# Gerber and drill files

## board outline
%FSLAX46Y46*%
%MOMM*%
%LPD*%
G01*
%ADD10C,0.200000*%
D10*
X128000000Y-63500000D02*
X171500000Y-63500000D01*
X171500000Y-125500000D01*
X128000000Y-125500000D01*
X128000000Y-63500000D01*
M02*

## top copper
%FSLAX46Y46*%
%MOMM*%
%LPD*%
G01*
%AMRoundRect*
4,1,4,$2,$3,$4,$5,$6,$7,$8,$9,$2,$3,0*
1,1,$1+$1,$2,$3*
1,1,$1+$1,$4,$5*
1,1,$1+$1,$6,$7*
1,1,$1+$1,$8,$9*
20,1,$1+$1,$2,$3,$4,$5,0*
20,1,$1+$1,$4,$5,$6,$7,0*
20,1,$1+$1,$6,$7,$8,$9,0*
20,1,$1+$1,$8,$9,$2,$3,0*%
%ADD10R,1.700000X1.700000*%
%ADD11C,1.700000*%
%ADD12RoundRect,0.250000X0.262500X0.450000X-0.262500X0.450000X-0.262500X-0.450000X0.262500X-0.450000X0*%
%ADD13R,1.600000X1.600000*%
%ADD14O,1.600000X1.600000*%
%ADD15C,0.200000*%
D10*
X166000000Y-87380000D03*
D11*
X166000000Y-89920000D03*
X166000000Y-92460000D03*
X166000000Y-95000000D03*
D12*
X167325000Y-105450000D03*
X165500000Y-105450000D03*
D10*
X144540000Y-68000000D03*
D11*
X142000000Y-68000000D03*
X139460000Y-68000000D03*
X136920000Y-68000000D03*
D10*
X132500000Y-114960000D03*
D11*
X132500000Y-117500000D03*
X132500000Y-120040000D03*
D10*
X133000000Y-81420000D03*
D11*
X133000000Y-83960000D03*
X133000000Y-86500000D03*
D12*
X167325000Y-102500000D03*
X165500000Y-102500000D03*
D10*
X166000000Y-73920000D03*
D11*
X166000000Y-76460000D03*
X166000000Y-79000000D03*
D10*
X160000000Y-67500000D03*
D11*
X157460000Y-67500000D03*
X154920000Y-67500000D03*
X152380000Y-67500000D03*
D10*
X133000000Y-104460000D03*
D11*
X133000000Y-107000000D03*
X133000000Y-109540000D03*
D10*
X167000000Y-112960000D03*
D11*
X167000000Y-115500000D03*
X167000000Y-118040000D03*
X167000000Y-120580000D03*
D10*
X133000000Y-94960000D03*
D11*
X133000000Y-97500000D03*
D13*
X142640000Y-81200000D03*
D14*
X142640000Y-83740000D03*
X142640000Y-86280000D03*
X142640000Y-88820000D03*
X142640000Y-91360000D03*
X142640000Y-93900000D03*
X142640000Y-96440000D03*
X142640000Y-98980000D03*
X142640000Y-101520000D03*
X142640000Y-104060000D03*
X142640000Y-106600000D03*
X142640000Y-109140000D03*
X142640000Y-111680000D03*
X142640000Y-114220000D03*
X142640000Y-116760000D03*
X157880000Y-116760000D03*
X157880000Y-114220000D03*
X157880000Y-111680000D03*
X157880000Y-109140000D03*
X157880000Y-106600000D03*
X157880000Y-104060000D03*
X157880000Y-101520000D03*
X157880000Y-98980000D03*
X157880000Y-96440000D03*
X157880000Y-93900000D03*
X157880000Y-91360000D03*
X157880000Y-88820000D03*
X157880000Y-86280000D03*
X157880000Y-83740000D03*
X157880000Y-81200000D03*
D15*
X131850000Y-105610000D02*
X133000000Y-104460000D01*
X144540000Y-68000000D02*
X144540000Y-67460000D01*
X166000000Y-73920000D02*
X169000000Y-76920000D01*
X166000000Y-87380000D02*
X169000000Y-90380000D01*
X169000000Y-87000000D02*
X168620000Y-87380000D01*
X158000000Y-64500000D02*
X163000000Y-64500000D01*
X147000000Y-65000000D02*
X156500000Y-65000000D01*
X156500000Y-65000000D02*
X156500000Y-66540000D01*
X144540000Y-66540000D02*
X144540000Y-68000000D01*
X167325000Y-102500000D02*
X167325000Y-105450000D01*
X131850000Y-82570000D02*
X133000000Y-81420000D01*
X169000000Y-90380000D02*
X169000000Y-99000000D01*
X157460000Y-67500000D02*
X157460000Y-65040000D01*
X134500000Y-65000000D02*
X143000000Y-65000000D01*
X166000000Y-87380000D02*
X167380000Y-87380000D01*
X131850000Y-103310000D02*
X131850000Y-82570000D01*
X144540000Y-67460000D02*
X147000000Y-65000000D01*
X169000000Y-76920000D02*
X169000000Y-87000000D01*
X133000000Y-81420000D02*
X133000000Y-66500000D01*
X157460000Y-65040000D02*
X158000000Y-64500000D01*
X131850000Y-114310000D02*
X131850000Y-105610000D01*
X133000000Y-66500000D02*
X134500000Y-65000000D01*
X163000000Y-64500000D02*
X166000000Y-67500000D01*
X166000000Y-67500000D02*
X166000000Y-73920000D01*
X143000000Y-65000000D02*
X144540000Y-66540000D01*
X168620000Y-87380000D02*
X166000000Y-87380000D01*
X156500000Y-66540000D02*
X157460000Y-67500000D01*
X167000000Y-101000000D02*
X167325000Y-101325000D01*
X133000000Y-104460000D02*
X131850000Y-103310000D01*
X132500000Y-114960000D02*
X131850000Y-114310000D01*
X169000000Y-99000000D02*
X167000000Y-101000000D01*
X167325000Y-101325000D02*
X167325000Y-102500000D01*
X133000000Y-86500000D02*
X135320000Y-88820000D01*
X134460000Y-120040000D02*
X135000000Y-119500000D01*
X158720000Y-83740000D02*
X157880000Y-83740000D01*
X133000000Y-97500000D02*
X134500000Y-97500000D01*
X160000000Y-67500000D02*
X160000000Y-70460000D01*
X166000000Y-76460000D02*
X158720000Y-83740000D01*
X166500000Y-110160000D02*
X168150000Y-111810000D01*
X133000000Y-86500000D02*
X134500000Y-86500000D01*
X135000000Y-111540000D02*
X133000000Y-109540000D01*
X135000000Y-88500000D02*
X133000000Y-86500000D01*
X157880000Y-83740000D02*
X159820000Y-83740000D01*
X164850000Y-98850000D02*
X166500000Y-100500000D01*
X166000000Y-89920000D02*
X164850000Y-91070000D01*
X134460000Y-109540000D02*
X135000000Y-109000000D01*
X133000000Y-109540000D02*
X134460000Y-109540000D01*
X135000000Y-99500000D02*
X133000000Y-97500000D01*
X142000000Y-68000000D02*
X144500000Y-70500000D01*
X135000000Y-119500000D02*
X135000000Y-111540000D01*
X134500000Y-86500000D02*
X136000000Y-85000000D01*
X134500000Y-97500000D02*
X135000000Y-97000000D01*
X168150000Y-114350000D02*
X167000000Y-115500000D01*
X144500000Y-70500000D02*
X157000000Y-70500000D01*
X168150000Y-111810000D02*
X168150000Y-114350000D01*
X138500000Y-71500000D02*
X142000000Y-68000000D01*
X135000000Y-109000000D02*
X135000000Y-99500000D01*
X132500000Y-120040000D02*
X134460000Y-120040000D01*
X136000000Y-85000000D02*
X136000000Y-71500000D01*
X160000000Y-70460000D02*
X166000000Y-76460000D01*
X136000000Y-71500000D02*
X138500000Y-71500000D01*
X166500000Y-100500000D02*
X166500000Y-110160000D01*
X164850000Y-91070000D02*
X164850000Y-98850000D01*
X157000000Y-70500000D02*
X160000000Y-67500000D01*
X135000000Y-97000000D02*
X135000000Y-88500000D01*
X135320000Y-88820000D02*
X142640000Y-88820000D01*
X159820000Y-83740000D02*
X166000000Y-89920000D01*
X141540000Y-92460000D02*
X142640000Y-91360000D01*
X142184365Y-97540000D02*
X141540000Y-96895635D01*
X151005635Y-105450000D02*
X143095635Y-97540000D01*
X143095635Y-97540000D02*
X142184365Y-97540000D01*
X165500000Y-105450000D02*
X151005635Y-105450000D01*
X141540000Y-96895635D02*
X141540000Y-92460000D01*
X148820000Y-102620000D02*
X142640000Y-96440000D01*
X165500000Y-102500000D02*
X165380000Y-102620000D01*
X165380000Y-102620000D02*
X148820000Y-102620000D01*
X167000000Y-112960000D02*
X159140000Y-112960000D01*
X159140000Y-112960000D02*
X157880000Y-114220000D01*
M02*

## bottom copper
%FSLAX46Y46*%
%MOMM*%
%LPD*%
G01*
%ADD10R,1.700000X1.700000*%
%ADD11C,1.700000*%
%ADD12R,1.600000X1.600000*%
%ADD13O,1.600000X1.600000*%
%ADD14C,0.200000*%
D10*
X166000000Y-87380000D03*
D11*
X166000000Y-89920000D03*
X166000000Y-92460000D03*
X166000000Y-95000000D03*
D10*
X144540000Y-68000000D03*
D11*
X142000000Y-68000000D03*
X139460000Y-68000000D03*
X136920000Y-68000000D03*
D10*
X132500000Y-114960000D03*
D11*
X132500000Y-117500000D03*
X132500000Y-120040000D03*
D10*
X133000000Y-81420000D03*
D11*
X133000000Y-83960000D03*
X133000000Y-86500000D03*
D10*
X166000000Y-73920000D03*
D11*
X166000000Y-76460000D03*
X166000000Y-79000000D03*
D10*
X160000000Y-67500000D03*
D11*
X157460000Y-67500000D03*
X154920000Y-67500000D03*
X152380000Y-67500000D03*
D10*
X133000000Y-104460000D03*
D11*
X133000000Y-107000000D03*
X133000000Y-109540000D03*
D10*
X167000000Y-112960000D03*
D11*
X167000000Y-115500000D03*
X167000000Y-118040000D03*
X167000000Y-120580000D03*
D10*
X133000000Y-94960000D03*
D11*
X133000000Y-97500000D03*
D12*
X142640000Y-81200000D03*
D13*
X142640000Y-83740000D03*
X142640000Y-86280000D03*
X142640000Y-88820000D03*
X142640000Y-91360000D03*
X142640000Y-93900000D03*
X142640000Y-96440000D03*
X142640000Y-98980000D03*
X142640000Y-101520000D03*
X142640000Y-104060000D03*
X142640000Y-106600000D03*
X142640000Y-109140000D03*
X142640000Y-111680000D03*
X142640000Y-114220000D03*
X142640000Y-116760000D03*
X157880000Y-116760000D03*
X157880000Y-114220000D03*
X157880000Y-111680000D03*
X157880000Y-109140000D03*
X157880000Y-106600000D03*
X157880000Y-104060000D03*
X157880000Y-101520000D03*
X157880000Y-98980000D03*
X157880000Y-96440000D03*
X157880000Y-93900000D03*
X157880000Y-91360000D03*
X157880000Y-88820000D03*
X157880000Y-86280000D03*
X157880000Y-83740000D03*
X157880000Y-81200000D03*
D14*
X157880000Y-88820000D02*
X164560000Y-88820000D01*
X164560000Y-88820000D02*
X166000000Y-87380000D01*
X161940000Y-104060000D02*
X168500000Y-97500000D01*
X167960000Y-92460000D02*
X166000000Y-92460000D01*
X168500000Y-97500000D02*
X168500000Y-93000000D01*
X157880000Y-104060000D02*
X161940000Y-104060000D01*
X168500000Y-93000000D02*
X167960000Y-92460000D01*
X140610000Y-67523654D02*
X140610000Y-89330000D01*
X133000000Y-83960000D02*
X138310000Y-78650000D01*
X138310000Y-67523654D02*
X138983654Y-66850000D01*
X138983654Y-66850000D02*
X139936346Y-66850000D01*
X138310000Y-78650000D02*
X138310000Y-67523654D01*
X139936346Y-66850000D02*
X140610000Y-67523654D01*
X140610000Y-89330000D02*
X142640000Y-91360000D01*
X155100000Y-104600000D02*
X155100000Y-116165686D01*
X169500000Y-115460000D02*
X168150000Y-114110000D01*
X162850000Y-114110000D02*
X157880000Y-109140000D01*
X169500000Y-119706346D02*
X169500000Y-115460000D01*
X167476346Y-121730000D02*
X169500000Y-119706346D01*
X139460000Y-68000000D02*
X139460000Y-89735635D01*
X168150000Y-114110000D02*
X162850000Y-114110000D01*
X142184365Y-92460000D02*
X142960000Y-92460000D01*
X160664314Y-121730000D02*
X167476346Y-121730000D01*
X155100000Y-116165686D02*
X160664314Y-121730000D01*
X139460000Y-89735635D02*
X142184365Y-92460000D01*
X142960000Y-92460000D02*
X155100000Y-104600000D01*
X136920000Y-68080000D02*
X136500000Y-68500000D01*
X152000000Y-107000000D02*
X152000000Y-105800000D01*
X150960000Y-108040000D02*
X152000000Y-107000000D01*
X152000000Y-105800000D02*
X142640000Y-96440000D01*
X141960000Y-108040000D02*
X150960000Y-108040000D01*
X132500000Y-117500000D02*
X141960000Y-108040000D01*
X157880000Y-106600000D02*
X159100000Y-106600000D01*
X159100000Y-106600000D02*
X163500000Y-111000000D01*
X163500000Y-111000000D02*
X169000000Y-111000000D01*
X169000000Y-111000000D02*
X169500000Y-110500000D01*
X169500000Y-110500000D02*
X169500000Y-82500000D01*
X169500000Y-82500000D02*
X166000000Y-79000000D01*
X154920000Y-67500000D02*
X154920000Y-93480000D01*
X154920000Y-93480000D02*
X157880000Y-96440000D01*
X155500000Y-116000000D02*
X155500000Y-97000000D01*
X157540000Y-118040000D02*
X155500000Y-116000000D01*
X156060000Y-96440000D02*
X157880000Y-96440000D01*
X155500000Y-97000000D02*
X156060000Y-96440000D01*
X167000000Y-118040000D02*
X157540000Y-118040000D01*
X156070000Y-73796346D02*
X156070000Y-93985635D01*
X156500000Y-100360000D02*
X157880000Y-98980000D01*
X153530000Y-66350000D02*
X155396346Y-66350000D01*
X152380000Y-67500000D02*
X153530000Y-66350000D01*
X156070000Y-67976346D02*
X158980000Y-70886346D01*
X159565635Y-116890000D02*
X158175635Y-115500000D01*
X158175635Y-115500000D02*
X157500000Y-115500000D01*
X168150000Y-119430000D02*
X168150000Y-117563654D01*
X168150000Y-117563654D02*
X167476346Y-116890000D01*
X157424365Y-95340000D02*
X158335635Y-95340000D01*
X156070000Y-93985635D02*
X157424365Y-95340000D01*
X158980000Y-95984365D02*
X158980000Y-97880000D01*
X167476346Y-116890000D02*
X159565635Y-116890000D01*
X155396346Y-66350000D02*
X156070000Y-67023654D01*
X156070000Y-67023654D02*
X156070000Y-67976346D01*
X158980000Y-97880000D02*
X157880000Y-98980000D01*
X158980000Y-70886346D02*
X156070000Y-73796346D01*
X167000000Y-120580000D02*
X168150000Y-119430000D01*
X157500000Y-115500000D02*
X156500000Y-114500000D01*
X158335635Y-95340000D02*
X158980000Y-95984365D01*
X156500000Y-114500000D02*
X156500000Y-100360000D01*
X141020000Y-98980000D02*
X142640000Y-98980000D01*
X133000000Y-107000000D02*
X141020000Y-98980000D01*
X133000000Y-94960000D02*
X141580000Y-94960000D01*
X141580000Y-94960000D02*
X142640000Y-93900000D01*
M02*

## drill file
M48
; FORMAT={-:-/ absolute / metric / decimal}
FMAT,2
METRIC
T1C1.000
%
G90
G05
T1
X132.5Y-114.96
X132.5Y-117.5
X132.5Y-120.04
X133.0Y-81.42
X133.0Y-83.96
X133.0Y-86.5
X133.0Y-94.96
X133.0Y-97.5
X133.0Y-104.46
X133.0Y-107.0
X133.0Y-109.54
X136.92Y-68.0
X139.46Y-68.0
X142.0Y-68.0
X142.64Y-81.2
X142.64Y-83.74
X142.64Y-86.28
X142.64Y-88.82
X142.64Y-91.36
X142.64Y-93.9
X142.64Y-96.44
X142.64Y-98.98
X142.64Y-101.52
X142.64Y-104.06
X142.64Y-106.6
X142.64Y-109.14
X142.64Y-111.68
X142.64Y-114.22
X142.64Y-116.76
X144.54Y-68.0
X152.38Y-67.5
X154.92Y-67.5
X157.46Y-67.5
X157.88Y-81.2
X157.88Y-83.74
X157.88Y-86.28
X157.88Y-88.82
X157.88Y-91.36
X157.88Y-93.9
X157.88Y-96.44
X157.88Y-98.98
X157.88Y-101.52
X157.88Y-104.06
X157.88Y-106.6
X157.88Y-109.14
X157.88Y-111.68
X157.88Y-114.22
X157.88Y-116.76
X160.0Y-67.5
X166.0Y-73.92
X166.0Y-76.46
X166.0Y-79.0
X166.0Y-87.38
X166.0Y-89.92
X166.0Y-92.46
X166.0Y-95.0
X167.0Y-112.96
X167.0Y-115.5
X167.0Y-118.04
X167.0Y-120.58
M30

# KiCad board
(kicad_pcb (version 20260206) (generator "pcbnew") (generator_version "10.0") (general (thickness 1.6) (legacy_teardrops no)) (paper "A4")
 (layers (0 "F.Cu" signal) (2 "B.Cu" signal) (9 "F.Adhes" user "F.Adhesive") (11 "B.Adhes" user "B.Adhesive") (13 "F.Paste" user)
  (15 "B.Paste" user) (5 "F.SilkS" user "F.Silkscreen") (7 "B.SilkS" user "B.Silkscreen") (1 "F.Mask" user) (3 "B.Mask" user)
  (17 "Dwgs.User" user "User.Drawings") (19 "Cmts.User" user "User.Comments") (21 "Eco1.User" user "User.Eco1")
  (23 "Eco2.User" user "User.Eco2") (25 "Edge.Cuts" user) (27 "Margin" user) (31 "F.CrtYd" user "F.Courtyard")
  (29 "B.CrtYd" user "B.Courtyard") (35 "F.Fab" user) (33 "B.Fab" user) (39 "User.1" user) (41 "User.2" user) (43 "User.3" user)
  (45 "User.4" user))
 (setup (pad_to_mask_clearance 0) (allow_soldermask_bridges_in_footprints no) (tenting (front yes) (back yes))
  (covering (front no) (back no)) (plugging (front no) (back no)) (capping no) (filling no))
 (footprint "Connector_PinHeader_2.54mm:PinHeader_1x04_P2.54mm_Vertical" (layer "F.Cu") (at 166 87.38)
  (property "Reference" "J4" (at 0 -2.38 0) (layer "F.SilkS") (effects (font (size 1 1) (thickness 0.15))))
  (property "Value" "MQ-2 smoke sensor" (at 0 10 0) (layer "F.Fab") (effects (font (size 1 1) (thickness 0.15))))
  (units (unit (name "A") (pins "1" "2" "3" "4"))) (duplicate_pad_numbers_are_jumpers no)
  (pad "1" thru_hole rect (at 0 0) (size 1.7 1.7) (drill 1) (layers "*.Cu" "*.Mask") (remove_unused_layers no) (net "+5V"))
  (pad "2" thru_hole circle (at 0 2.54) (size 1.7 1.7) (drill 1) (layers "*.Cu" "*.Mask") (remove_unused_layers no) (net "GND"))
  (pad "3" thru_hole circle (at 0 5.08) (size 1.7 1.7) (drill 1) (layers "*.Cu" "*.Mask") (remove_unused_layers no) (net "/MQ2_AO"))
  (pad "4" thru_hole circle (at 0 7.62) (size 1.7 1.7) (drill 1) (layers "*.Cu" "*.Mask") (remove_unused_layers no)
   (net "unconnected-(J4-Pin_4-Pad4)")))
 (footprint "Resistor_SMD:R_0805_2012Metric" (layer "F.Cu") (at 166.4125 105.45 180)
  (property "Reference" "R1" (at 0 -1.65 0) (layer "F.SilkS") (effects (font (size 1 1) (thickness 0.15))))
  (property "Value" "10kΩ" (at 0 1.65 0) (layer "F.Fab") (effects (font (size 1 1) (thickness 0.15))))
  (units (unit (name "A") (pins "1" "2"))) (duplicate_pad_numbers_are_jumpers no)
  (pad "1" smd roundrect (at -0.9125 0 180) (size 1.025 1.4) (layers "F.Cu" "F.Mask" "F.Paste") (roundrect_rratio 0.243902) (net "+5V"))
  (pad "2" smd roundrect (at 0.9125 0 180) (size 1.025 1.4) (layers "F.Cu" "F.Mask" "F.Paste") (roundrect_rratio 0.243902) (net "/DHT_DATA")))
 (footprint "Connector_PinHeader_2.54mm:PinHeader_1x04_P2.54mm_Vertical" (layer "F.Cu") (at 144.54 68 -90)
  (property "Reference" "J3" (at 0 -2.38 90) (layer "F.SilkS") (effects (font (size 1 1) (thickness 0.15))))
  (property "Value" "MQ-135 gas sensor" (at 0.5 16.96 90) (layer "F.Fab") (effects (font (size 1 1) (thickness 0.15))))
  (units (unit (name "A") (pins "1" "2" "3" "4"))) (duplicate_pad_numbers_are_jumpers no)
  (pad "1" thru_hole rect (at 0 0 270) (size 1.7 1.7) (drill 1) (layers "*.Cu" "*.Mask") (remove_unused_layers no) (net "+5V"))
  (pad "2" thru_hole circle (at 0 2.54 270) (size 1.7 1.7) (drill 1) (layers "*.Cu" "*.Mask") (remove_unused_layers no) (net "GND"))
  (pad "3" thru_hole circle (at 0 5.08 270) (size 1.7 1.7) (drill 1) (layers "*.Cu" "*.Mask") (remove_unused_layers no) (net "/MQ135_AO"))
  (pad "4" thru_hole circle (at 0 7.62 270) (size 1.7 1.7) (drill 1) (layers "*.Cu" "*.Mask") (remove_unused_layers no)
   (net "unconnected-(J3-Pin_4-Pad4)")))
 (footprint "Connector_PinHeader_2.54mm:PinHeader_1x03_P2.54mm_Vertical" (layer "F.Cu") (at 132.5 114.96)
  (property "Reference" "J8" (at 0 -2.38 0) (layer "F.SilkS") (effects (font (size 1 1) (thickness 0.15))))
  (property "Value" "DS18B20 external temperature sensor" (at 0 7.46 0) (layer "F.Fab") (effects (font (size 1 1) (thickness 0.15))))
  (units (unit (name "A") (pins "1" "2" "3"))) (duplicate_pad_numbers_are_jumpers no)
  (pad "1" thru_hole rect (at 0 0) (size 1.7 1.7) (drill 1) (layers "*.Cu" "*.Mask") (remove_unused_layers no) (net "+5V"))
  (pad "2" thru_hole circle (at 0 2.54) (size 1.7 1.7) (drill 1) (layers "*.Cu" "*.Mask") (remove_unused_layers no) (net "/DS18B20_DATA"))
  (pad "3" thru_hole circle (at 0 5.08) (size 1.7 1.7) (drill 1) (layers "*.Cu" "*.Mask") (remove_unused_layers no) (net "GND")))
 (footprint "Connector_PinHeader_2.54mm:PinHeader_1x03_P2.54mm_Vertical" (layer "F.Cu") (at 133 81.42)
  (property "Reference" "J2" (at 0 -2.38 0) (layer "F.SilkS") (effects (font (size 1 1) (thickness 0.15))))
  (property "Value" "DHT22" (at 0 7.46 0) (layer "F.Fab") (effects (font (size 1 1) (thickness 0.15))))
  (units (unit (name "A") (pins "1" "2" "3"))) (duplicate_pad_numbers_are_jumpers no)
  (pad "1" thru_hole rect (at 0 0) (size 1.7 1.7) (drill 1) (layers "*.Cu" "*.Mask") (remove_unused_layers no) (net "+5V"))
  (pad "2" thru_hole circle (at 0 2.54) (size 1.7 1.7) (drill 1) (layers "*.Cu" "*.Mask") (remove_unused_layers no) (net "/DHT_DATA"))
  (pad "3" thru_hole circle (at 0 5.08) (size 1.7 1.7) (drill 1) (layers "*.Cu" "*.Mask") (remove_unused_layers no) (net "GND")))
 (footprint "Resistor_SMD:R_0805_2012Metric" (layer "F.Cu") (at 166.4125 102.5 180)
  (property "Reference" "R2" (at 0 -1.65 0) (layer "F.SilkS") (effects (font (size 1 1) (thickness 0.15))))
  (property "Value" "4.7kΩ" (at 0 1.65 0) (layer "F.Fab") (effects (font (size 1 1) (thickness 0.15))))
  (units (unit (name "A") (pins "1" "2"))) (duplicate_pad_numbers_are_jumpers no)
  (pad "1" smd roundrect (at -0.9125 0 180) (size 1.025 1.4) (layers "F.Cu" "F.Mask" "F.Paste") (roundrect_rratio 0.243902) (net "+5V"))
  (pad "2" smd roundrect (at 0.9125 0 180) (size 1.025 1.4) (layers "F.Cu" "F.Mask" "F.Paste") (roundrect_rratio 0.243902)
   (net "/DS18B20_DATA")))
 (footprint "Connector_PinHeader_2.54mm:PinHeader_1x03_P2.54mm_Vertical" (layer "F.Cu") (at 166 73.92)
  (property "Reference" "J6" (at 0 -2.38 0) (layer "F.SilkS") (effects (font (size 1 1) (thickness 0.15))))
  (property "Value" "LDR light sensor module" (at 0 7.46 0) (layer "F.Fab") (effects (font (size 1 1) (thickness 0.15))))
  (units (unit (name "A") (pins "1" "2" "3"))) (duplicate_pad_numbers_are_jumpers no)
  (pad "1" thru_hole rect (at 0 0) (size 1.7 1.7) (drill 1) (layers "*.Cu" "*.Mask") (remove_unused_layers no) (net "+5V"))
  (pad "2" thru_hole circle (at 0 2.54) (size 1.7 1.7) (drill 1) (layers "*.Cu" "*.Mask") (remove_unused_layers no) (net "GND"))
  (pad "3" thru_hole circle (at 0 5.08) (size 1.7 1.7) (drill 1) (layers "*.Cu" "*.Mask") (remove_unused_layers no) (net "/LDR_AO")))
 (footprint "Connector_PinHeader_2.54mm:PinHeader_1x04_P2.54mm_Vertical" (layer "F.Cu") (at 160 67.5 -90)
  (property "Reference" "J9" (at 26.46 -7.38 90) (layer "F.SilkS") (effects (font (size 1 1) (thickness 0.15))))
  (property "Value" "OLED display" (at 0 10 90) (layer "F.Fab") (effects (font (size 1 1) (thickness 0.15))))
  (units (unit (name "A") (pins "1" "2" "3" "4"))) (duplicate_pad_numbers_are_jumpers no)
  (pad "1" thru_hole rect (at 0 0 270) (size 1.7 1.7) (drill 1) (layers "*.Cu" "*.Mask") (remove_unused_layers no) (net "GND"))
  (pad "2" thru_hole circle (at 0 2.54 270) (size 1.7 1.7) (drill 1) (layers "*.Cu" "*.Mask") (remove_unused_layers no) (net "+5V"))
  (pad "3" thru_hole circle (at 0 5.08 270) (size 1.7 1.7) (drill 1) (layers "*.Cu" "*.Mask") (remove_unused_layers no) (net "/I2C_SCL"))
  (pad "4" thru_hole circle (at 0 7.62 270) (size 1.7 1.7) (drill 1) (layers "*.Cu" "*.Mask") (remove_unused_layers no) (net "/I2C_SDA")))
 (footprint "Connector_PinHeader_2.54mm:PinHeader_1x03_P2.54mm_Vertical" (layer "F.Cu") (at 133 104.46)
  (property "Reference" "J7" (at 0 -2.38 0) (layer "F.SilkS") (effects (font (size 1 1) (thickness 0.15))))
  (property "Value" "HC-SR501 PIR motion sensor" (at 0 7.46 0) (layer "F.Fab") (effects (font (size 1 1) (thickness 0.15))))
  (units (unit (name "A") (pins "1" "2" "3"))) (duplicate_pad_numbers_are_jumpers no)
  (pad "1" thru_hole rect (at 0 0) (size 1.7 1.7) (drill 1) (layers "*.Cu" "*.Mask") (remove_unused_layers no) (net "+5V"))
  (pad "2" thru_hole circle (at 0 2.54) (size 1.7 1.7) (drill 1) (layers "*.Cu" "*.Mask") (remove_unused_layers no) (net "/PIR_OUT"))
  (pad "3" thru_hole circle (at 0 5.08) (size 1.7 1.7) (drill 1) (layers "*.Cu" "*.Mask") (remove_unused_layers no) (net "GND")))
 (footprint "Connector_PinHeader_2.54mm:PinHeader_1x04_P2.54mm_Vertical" (layer "F.Cu") (at 167 112.96)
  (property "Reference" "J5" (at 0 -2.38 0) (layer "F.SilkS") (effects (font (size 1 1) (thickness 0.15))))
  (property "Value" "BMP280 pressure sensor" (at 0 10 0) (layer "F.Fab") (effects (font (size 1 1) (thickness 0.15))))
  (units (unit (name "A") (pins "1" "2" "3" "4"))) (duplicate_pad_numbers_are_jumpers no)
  (pad "1" thru_hole rect (at 0 0) (size 1.7 1.7) (drill 1) (layers "*.Cu" "*.Mask") (remove_unused_layers no) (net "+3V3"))
  (pad "2" thru_hole circle (at 0 2.54) (size 1.7 1.7) (drill 1) (layers "*.Cu" "*.Mask") (remove_unused_layers no) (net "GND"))
  (pad "3" thru_hole circle (at 0 5.08) (size 1.7 1.7) (drill 1) (layers "*.Cu" "*.Mask") (remove_unused_layers no) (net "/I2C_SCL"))
  (pad "4" thru_hole circle (at 0 7.62) (size 1.7 1.7) (drill 1) (layers "*.Cu" "*.Mask") (remove_unused_layers no) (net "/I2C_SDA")))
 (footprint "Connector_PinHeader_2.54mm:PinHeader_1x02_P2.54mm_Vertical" (layer "F.Cu") (at 133 94.96)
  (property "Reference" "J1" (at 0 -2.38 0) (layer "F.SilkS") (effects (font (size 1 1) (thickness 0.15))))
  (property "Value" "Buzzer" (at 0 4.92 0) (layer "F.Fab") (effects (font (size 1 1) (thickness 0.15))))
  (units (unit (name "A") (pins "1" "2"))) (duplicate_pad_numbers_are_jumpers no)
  (pad "1" thru_hole rect (at 0 0) (size 1.7 1.7) (drill 1) (layers "*.Cu" "*.Mask") (remove_unused_layers no) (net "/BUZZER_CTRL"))
  (pad "2" thru_hole circle (at 0 2.54) (size 1.7 1.7) (drill 1) (layers "*.Cu" "*.Mask") (remove_unused_layers no) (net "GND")))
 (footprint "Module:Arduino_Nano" (layer "F.Cu") (at 142.64 81.2)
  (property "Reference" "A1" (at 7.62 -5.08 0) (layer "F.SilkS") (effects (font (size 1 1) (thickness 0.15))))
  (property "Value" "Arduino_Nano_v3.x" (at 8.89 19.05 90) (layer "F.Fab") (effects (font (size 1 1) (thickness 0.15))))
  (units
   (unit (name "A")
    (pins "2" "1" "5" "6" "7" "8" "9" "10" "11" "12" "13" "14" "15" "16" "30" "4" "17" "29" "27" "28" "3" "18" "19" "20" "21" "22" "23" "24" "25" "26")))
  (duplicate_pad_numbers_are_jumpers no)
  (pad "1" thru_hole rect (at 0 0) (size 1.6 1.6) (drill 1) (layers "*.Cu" "*.Mask") (remove_unused_layers no)
   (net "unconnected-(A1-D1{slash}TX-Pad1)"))
  (pad "2" thru_hole oval (at 0 2.54) (size 1.6 1.6) (drill 1) (layers "*.Cu" "*.Mask") (remove_unused_layers no)
   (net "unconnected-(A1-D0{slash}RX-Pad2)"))
  (pad "3" thru_hole oval (at 0 5.08) (size 1.6 1.6) (drill 1) (layers "*.Cu" "*.Mask") (remove_unused_layers no)
   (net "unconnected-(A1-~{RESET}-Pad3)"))
  (pad "4" thru_hole oval (at 0 7.62) (size 1.6 1.6) (drill 1) (layers "*.Cu" "*.Mask") (remove_unused_layers no) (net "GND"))
  (pad "5" thru_hole oval (at 0 10.16) (size 1.6 1.6) (drill 1) (layers "*.Cu" "*.Mask") (remove_unused_layers no) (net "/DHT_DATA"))
  (pad "6" thru_hole oval (at 0 12.7) (size 1.6 1.6) (drill 1) (layers "*.Cu" "*.Mask") (remove_unused_layers no) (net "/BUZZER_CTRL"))
  (pad "7" thru_hole oval (at 0 15.24) (size 1.6 1.6) (drill 1) (layers "*.Cu" "*.Mask") (remove_unused_layers no) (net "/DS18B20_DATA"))
  (pad "8" thru_hole oval (at 0 17.78) (size 1.6 1.6) (drill 1) (layers "*.Cu" "*.Mask") (remove_unused_layers no) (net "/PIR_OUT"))
  (pad "9" thru_hole oval (at 0 20.32) (size 1.6 1.6) (drill 1) (layers "*.Cu" "*.Mask") (remove_unused_layers no)
   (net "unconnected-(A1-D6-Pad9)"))
  (pad "10" thru_hole oval (at 0 22.86) (size 1.6 1.6) (drill 1) (layers "*.Cu" "*.Mask") (remove_unused_layers no)
   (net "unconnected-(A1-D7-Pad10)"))
  (pad "11" thru_hole oval (at 0 25.4) (size 1.6 1.6) (drill 1) (layers "*.Cu" "*.Mask") (remove_unused_layers no)
   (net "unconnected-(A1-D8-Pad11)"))
  (pad "12" thru_hole oval (at 0 27.94) (size 1.6 1.6) (drill 1) (layers "*.Cu" "*.Mask") (remove_unused_layers no)
   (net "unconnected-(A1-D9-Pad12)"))
  (pad "13" thru_hole oval (at 0 30.48) (size 1.6 1.6) (drill 1) (layers "*.Cu" "*.Mask") (remove_unused_layers no)
   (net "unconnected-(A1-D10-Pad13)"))
  (pad "14" thru_hole oval (at 0 33.02) (size 1.6 1.6) (drill 1) (layers "*.Cu" "*.Mask") (remove_unused_layers no)
   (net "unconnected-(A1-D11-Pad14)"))
  (pad "15" thru_hole oval (at 0 35.56) (size 1.6 1.6) (drill 1) (layers "*.Cu" "*.Mask") (remove_unused_layers no)
   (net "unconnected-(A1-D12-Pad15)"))
  (pad "16" thru_hole oval (at 15.24 35.56) (size 1.6 1.6) (drill 1) (layers "*.Cu" "*.Mask") (remove_unused_layers no)
   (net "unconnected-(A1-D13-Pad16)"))
  (pad "17" thru_hole oval (at 15.24 33.02) (size 1.6 1.6) (drill 1) (layers "*.Cu" "*.Mask") (remove_unused_layers no) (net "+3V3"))
  (pad "18" thru_hole oval (at 15.24 30.48) (size 1.6 1.6) (drill 1) (layers "*.Cu" "*.Mask") (remove_unused_layers no)
   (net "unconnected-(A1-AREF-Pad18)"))
  (pad "19" thru_hole oval (at 15.24 27.94) (size 1.6 1.6) (drill 1) (layers "*.Cu" "*.Mask") (remove_unused_layers no) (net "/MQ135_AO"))
  (pad "20" thru_hole oval (at 15.24 25.4) (size 1.6 1.6) (drill 1) (layers "*.Cu" "*.Mask") (remove_unused_layers no) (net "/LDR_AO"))
  (pad "21" thru_hole oval (at 15.24 22.86) (size 1.6 1.6) (drill 1) (layers "*.Cu" "*.Mask") (remove_unused_layers no) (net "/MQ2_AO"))
  (pad "22" thru_hole oval (at 15.24 20.32) (size 1.6 1.6) (drill 1) (layers "*.Cu" "*.Mask") (remove_unused_layers no)
   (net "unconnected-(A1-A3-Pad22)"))
  (pad "23" thru_hole oval (at 15.24 17.78) (size 1.6 1.6) (drill 1) (layers "*.Cu" "*.Mask") (remove_unused_layers no) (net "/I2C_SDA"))
  (pad "24" thru_hole oval (at 15.24 15.24) (size 1.6 1.6) (drill 1) (layers "*.Cu" "*.Mask") (remove_unused_layers no) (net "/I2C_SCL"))
  (pad "25" thru_hole oval (at 15.24 12.7) (size 1.6 1.6) (drill 1) (layers "*.Cu" "*.Mask") (remove_unused_layers no)
   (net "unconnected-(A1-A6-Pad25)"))
  (pad "26" thru_hole oval (at 15.24 10.16) (size 1.6 1.6) (drill 1) (layers "*.Cu" "*.Mask") (remove_unused_layers no)
   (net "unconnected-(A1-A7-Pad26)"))
  (pad "27" thru_hole oval (at 15.24 7.62) (size 1.6 1.6) (drill 1) (layers "*.Cu" "*.Mask") (remove_unused_layers no) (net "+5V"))
  (pad "28" thru_hole oval (at 15.24 5.08) (size 1.6 1.6) (drill 1) (layers "*.Cu" "*.Mask") (remove_unused_layers no)
   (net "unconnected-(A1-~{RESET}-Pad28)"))
  (pad "29" thru_hole oval (at 15.24 2.54) (size 1.6 1.6) (drill 1) (layers "*.Cu" "*.Mask") (remove_unused_layers no) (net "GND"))
  (pad "30" thru_hole oval (at 15.24 0) (size 1.6 1.6) (drill 1) (layers "*.Cu" "*.Mask") (remove_unused_layers no)
   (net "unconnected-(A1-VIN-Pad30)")))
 (gr_rect (start 128 63.5) (end 171.5 125.5) (stroke (width 0.2) (type solid)) (fill no) (layer "Edge.Cuts"))
 (segment (start 131.85 105.61) (end 133 104.46) (width 0.2) (layer "F.Cu") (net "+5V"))
 (segment (start 144.54 68) (end 144.54 67.46) (width 0.2) (layer "F.Cu") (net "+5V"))
 (segment (start 166 73.92) (end 169 76.92) (width 0.2) (layer "F.Cu") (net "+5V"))
 (segment (start 166 87.38) (end 169 90.38) (width 0.2) (layer "F.Cu") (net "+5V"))
 (segment (start 169 87) (end 168.62 87.38) (width 0.2) (layer "F.Cu") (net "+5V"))
 (segment (start 158 64.5) (end 163 64.5) (width 0.2) (layer "F.Cu") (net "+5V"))
 (segment (start 147 65) (end 156.5 65) (width 0.2) (layer "F.Cu") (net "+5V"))
 (segment (start 156.5 65) (end 156.5 66.54) (width 0.2) (layer "F.Cu") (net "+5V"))
 (segment (start 144.54 66.54) (end 144.54 68) (width 0.2) (layer "F.Cu") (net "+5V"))
 (segment (start 167.325 102.5) (end 167.325 105.45) (width 0.2) (layer "F.Cu") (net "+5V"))
 (segment (start 131.85 82.57) (end 133 81.42) (width 0.2) (layer "F.Cu") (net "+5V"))
 (segment (start 169 90.38) (end 169 99) (width 0.2) (layer "F.Cu") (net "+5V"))
 (segment (start 157.46 67.5) (end 157.46 65.04) (width 0.2) (layer "F.Cu") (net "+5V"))
 (segment (start 134.5 65) (end 143 65) (width 0.2) (layer "F.Cu") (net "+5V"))
 (segment (start 166 87.38) (end 167.38 87.38) (width 0.2) (layer "F.Cu") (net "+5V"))
 (segment (start 131.85 103.31) (end 131.85 82.57) (width 0.2) (layer "F.Cu") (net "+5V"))
 (segment (start 144.54 67.46) (end 147 65) (width 0.2) (layer "F.Cu") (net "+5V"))
 (segment (start 169 76.92) (end 169 87) (width 0.2) (layer "F.Cu") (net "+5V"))
 (segment (start 133 81.42) (end 133 66.5) (width 0.2) (layer "F.Cu") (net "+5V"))
 (segment (start 157.46 65.04) (end 158 64.5) (width 0.2) (layer "F.Cu") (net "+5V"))
 (segment (start 131.85 114.31) (end 131.85 105.61) (width 0.2) (layer "F.Cu") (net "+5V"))
 (segment (start 133 66.5) (end 134.5 65) (width 0.2) (layer "F.Cu") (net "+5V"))
 (segment (start 163 64.5) (end 166 67.5) (width 0.2) (layer "F.Cu") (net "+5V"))
 (segment (start 166 67.5) (end 166 73.92) (width 0.2) (layer "F.Cu") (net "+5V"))
 (segment (start 143 65) (end 144.54 66.54) (width 0.2) (layer "F.Cu") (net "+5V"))
 (segment (start 168.62 87.38) (end 166 87.38) (width 0.2) (layer "F.Cu") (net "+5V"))
 (segment (start 156.5 66.54) (end 157.46 67.5) (width 0.2) (layer "F.Cu") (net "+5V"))
 (segment (start 167 101) (end 167.325 101.325) (width 0.2) (layer "F.Cu") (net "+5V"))
 (segment (start 133 104.46) (end 131.85 103.31) (width 0.2) (layer "F.Cu") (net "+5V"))
 (segment (start 132.5 114.96) (end 131.85 114.31) (width 0.2) (layer "F.Cu") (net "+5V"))
 (segment (start 169 99) (end 167 101) (width 0.2) (layer "F.Cu") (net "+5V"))
 (segment (start 167.325 101.325) (end 167.325 102.5) (width 0.2) (layer "F.Cu") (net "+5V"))
 (segment (start 157.88 88.82) (end 164.56 88.82) (width 0.2) (layer "B.Cu") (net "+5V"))
 (segment (start 164.56 88.82) (end 166 87.38) (width 0.2) (layer "B.Cu") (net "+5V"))
 (segment (start 133 86.5) (end 135.32 88.82) (width 0.2) (layer "F.Cu") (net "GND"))
 (segment (start 134.46 120.04) (end 135 119.5) (width 0.2) (layer "F.Cu") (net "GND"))
 (segment (start 158.72 83.74) (end 157.88 83.74) (width 0.2) (layer "F.Cu") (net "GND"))
 (segment (start 133 97.5) (end 134.5 97.5) (width 0.2) (layer "F.Cu") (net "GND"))
 (segment (start 160 67.5) (end 160 70.46) (width 0.2) (layer "F.Cu") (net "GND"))
 (segment (start 166 76.46) (end 158.72 83.74) (width 0.2) (layer "F.Cu") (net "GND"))
 (segment (start 166.5 110.16) (end 168.15 111.81) (width 0.2) (layer "F.Cu") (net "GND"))
 (segment (start 133 86.5) (end 134.5 86.5) (width 0.2) (layer "F.Cu") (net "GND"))
 (segment (start 135 111.54) (end 133 109.54) (width 0.2) (layer "F.Cu") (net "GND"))
 (segment (start 135 88.5) (end 133 86.5) (width 0.2) (layer "F.Cu") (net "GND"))
 (segment (start 157.88 83.74) (end 159.82 83.74) (width 0.2) (layer "F.Cu") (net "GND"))
 (segment (start 164.85 98.85) (end 166.5 100.5) (width 0.2) (layer "F.Cu") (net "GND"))
 (segment (start 166 89.92) (end 164.85 91.07) (width 0.2) (layer "F.Cu") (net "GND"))
 (segment (start 134.46 109.54) (end 135 109) (width 0.2) (layer "F.Cu") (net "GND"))
 (segment (start 133 109.54) (end 134.46 109.54) (width 0.2) (layer "F.Cu") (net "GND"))
 (segment (start 135 99.5) (end 133 97.5) (width 0.2) (layer "F.Cu") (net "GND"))
 (segment (start 142 68) (end 144.5 70.5) (width 0.2) (layer "F.Cu") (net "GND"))
 (segment (start 135 119.5) (end 135 111.54) (width 0.2) (layer "F.Cu") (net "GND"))
 (segment (start 134.5 86.5) (end 136 85) (width 0.2) (layer "F.Cu") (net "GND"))
 (segment (start 134.5 97.5) (end 135 97) (width 0.2) (layer "F.Cu") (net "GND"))
 (segment (start 168.15 114.35) (end 167 115.5) (width 0.2) (layer "F.Cu") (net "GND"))
 (segment (start 144.5 70.5) (end 157 70.5) (width 0.2) (layer "F.Cu") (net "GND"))
 (segment (start 168.15 111.81) (end 168.15 114.35) (width 0.2) (layer "F.Cu") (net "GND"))
 (segment (start 138.5 71.5) (end 142 68) (width 0.2) (layer "F.Cu") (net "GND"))
 (segment (start 135 109) (end 135 99.5) (width 0.2) (layer "F.Cu") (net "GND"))
 (segment (start 132.5 120.04) (end 134.46 120.04) (width 0.2) (layer "F.Cu") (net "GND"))
 (segment (start 136 85) (end 136 71.5) (width 0.2) (layer "F.Cu") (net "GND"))
 (segment (start 160 70.46) (end 166 76.46) (width 0.2) (layer "F.Cu") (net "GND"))
 (segment (start 136 71.5) (end 138.5 71.5) (width 0.2) (layer "F.Cu") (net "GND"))
 (segment (start 166.5 100.5) (end 166.5 110.16) (width 0.2) (layer "F.Cu") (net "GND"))
 (segment (start 164.85 91.07) (end 164.85 98.85) (width 0.2) (layer "F.Cu") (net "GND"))
 (segment (start 157 70.5) (end 160 67.5) (width 0.2) (layer "F.Cu") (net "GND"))
 (segment (start 135 97) (end 135 88.5) (width 0.2) (layer "F.Cu") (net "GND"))
 (segment (start 135.32 88.82) (end 142.64 88.82) (width 0.2) (layer "F.Cu") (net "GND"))
 (segment (start 159.82 83.74) (end 166 89.92) (width 0.2) (layer "F.Cu") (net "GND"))
 (segment (start 161.94 104.06) (end 168.5 97.5) (width 0.2) (layer "B.Cu") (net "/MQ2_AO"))
 (segment (start 167.96 92.46) (end 166 92.46) (width 0.2) (layer "B.Cu") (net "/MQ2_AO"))
 (segment (start 168.5 97.5) (end 168.5 93) (width 0.2) (layer "B.Cu") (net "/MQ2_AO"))
 (segment (start 157.88 104.06) (end 161.94 104.06) (width 0.2) (layer "B.Cu") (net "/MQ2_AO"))
 (segment (start 168.5 93) (end 167.96 92.46) (width 0.2) (layer "B.Cu") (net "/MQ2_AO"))
 (segment (start 141.54 92.46) (end 142.64 91.36) (width 0.2) (layer "F.Cu") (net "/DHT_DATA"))
 (segment (start 142.184365 97.54) (end 141.54 96.895635) (width 0.2) (layer "F.Cu") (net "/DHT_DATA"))
 (segment (start 151.005635 105.45) (end 143.095635 97.54) (width 0.2) (layer "F.Cu") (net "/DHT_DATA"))
 (segment (start 143.095635 97.54) (end 142.184365 97.54) (width 0.2) (layer "F.Cu") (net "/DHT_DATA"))
 (segment (start 165.5 105.45) (end 151.005635 105.45) (width 0.2) (layer "F.Cu") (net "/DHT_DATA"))
 (segment (start 141.54 96.895635) (end 141.54 92.46) (width 0.2) (layer "F.Cu") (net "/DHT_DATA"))
 (segment (start 140.61 67.523654) (end 140.61 89.33) (width 0.2) (layer "B.Cu") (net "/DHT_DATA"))
 (segment (start 133 83.96) (end 138.31 78.65) (width 0.2) (layer "B.Cu") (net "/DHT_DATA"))
 (segment (start 138.31 67.523654) (end 138.983654 66.85) (width 0.2) (layer "B.Cu") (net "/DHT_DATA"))
 (segment (start 138.983654 66.85) (end 139.936346 66.85) (width 0.2) (layer "B.Cu") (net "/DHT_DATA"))
 (segment (start 138.31 78.65) (end 138.31 67.523654) (width 0.2) (layer "B.Cu") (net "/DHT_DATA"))
 (segment (start 139.936346 66.85) (end 140.61 67.523654) (width 0.2) (layer "B.Cu") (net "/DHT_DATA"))
 (segment (start 140.61 89.33) (end 142.64 91.36) (width 0.2) (layer "B.Cu") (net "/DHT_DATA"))
 (segment (start 155.1 104.6) (end 155.1 116.165686) (width 0.2) (layer "B.Cu") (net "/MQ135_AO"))
 (segment (start 169.5 115.46) (end 168.15 114.11) (width 0.2) (layer "B.Cu") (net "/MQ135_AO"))
 (segment (start 162.85 114.11) (end 157.88 109.14) (width 0.2) (layer "B.Cu") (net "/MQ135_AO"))
 (segment (start 169.5 119.706346) (end 169.5 115.46) (width 0.2) (layer "B.Cu") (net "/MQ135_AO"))
 (segment (start 167.476346 121.73) (end 169.5 119.706346) (width 0.2) (layer "B.Cu") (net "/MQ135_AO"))
 (segment (start 139.46 68) (end 139.46 89.735635) (width 0.2) (layer "B.Cu") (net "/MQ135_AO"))
 (segment (start 168.15 114.11) (end 162.85 114.11) (width 0.2) (layer "B.Cu") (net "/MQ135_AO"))
 (segment (start 142.184365 92.46) (end 142.96 92.46) (width 0.2) (layer "B.Cu") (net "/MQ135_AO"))
 (segment (start 160.664314 121.73) (end 167.476346 121.73) (width 0.2) (layer "B.Cu") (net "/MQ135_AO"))
 (segment (start 155.1 116.165686) (end 160.664314 121.73) (width 0.2) (layer "B.Cu") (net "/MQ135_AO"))
 (segment (start 139.46 89.735635) (end 142.184365 92.46) (width 0.2) (layer "B.Cu") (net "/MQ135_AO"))
 (segment (start 142.96 92.46) (end 155.1 104.6) (width 0.2) (layer "B.Cu") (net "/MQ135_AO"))
 (segment (start 136.92 68.08) (end 136.5 68.5) (width 0.2) (layer "B.Cu") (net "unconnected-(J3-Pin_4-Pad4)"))
 (segment (start 148.82 102.62) (end 142.64 96.44) (width 0.2) (layer "F.Cu") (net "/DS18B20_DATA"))
 (segment (start 165.5 102.5) (end 165.38 102.62) (width 0.2) (layer "F.Cu") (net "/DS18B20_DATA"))
 (segment (start 165.38 102.62) (end 148.82 102.62) (width 0.2) (layer "F.Cu") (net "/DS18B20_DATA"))
 (segment (start 152 107) (end 152 105.8) (width 0.2) (layer "B.Cu") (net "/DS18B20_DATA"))
 (segment (start 150.96 108.04) (end 152 107) (width 0.2) (layer "B.Cu") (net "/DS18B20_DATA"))
 (segment (start 152 105.8) (end 142.64 96.44) (width 0.2) (layer "B.Cu") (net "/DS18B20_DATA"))
 (segment (start 141.96 108.04) (end 150.96 108.04) (width 0.2) (layer "B.Cu") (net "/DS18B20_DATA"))
 (segment (start 132.5 117.5) (end 141.96 108.04) (width 0.2) (layer "B.Cu") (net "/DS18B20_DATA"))
 (segment (start 157.88 106.6) (end 159.1 106.6) (width 0.2) (layer "B.Cu") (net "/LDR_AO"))
 (segment (start 159.1 106.6) (end 163.5 111) (width 0.2) (layer "B.Cu") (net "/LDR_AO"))
 (segment (start 163.5 111) (end 169 111) (width 0.2) (layer "B.Cu") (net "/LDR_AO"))
 (segment (start 169 111) (end 169.5 110.5) (width 0.2) (layer "B.Cu") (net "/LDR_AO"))
 (segment (start 169.5 110.5) (end 169.5 82.5) (width 0.2) (layer "B.Cu") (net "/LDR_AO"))
 (segment (start 169.5 82.5) (end 166 79) (width 0.2) (layer "B.Cu") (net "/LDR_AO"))
 (segment (start 154.92 67.5) (end 154.92 93.48) (width 0.2) (layer "B.Cu") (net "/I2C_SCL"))
 (segment (start 154.92 93.48) (end 157.88 96.44) (width 0.2) (layer "B.Cu") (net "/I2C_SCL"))
 (segment (start 155.5 116) (end 155.5 97) (width 0.2) (layer "B.Cu") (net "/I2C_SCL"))
 (segment (start 157.54 118.04) (end 155.5 116) (width 0.2) (layer "B.Cu") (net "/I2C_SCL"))
 (segment (start 156.06 96.44) (end 157.88 96.44) (width 0.2) (layer "B.Cu") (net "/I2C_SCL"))
 (segment (start 155.5 97) (end 156.06 96.44) (width 0.2) (layer "B.Cu") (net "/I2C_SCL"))
 (segment (start 167 118.04) (end 157.54 118.04) (width 0.2) (layer "B.Cu") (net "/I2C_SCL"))
 (segment (start 156.07 73.796346) (end 156.07 93.985635) (width 0.2) (layer "B.Cu") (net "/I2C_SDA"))
 (segment (start 156.5 100.36) (end 157.88 98.98) (width 0.2) (layer "B.Cu") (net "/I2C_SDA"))
 (segment (start 153.53 66.35) (end 155.396346 66.35) (width 0.2) (layer "B.Cu") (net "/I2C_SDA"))
 (segment (start 152.38 67.5) (end 153.53 66.35) (width 0.2) (layer "B.Cu") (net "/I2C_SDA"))
 (segment (start 156.07 67.976346) (end 158.98 70.886346) (width 0.2) (layer "B.Cu") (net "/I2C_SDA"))
 (segment (start 159.565635 116.89) (end 158.175635 115.5) (width 0.2) (layer "B.Cu") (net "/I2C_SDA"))
 (segment (start 158.175635 115.5) (end 157.5 115.5) (width 0.2) (layer "B.Cu") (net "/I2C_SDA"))
 (segment (start 168.15 119.43) (end 168.15 117.563654) (width 0.2) (layer "B.Cu") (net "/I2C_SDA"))
 (segment (start 168.15 117.563654) (end 167.476346 116.89) (width 0.2) (layer "B.Cu") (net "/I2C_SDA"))
 (segment (start 157.424365 95.34) (end 158.335635 95.34) (width 0.2) (layer "B.Cu") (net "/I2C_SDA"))
 (segment (start 156.07 93.985635) (end 157.424365 95.34) (width 0.2) (layer "B.Cu") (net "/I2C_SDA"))
 (segment (start 158.98 95.984365) (end 158.98 97.88) (width 0.2) (layer "B.Cu") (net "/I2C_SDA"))
 (segment (start 167.476346 116.89) (end 159.565635 116.89) (width 0.2) (layer "B.Cu") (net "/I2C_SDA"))
 (segment (start 155.396346 66.35) (end 156.07 67.023654) (width 0.2) (layer "B.Cu") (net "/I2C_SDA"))
 (segment (start 156.07 67.023654) (end 156.07 67.976346) (width 0.2) (layer "B.Cu") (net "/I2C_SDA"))
 (segment (start 158.98 97.88) (end 157.88 98.98) (width 0.2) (layer "B.Cu") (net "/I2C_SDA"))
 (segment (start 158.98 70.886346) (end 156.07 73.796346) (width 0.2) (layer "B.Cu") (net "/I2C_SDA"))
 (segment (start 167 120.58) (end 168.15 119.43) (width 0.2) (layer "B.Cu") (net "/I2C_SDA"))
 (segment (start 157.5 115.5) (end 156.5 114.5) (width 0.2) (layer "B.Cu") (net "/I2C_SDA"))
 (segment (start 158.335635 95.34) (end 158.98 95.984365) (width 0.2) (layer "B.Cu") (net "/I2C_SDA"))
 (segment (start 156.5 114.5) (end 156.5 100.36) (width 0.2) (layer "B.Cu") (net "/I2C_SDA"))
 (segment (start 141.02 98.98) (end 142.64 98.98) (width 0.2) (layer "B.Cu") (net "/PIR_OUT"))
 (segment (start 133 107) (end 141.02 98.98) (width 0.2) (layer "B.Cu") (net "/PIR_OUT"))
 (segment (start 167 112.96) (end 159.14 112.96) (width 0.2) (layer "F.Cu") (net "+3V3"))
 (segment (start 159.14 112.96) (end 157.88 114.22) (width 0.2) (layer "F.Cu") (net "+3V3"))
 (segment (start 133 94.96) (end 141.58 94.96) (width 0.2) (layer "B.Cu") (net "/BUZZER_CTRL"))
 (segment (start 141.58 94.96) (end 142.64 93.9) (width 0.2) (layer "B.Cu") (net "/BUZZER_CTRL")))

